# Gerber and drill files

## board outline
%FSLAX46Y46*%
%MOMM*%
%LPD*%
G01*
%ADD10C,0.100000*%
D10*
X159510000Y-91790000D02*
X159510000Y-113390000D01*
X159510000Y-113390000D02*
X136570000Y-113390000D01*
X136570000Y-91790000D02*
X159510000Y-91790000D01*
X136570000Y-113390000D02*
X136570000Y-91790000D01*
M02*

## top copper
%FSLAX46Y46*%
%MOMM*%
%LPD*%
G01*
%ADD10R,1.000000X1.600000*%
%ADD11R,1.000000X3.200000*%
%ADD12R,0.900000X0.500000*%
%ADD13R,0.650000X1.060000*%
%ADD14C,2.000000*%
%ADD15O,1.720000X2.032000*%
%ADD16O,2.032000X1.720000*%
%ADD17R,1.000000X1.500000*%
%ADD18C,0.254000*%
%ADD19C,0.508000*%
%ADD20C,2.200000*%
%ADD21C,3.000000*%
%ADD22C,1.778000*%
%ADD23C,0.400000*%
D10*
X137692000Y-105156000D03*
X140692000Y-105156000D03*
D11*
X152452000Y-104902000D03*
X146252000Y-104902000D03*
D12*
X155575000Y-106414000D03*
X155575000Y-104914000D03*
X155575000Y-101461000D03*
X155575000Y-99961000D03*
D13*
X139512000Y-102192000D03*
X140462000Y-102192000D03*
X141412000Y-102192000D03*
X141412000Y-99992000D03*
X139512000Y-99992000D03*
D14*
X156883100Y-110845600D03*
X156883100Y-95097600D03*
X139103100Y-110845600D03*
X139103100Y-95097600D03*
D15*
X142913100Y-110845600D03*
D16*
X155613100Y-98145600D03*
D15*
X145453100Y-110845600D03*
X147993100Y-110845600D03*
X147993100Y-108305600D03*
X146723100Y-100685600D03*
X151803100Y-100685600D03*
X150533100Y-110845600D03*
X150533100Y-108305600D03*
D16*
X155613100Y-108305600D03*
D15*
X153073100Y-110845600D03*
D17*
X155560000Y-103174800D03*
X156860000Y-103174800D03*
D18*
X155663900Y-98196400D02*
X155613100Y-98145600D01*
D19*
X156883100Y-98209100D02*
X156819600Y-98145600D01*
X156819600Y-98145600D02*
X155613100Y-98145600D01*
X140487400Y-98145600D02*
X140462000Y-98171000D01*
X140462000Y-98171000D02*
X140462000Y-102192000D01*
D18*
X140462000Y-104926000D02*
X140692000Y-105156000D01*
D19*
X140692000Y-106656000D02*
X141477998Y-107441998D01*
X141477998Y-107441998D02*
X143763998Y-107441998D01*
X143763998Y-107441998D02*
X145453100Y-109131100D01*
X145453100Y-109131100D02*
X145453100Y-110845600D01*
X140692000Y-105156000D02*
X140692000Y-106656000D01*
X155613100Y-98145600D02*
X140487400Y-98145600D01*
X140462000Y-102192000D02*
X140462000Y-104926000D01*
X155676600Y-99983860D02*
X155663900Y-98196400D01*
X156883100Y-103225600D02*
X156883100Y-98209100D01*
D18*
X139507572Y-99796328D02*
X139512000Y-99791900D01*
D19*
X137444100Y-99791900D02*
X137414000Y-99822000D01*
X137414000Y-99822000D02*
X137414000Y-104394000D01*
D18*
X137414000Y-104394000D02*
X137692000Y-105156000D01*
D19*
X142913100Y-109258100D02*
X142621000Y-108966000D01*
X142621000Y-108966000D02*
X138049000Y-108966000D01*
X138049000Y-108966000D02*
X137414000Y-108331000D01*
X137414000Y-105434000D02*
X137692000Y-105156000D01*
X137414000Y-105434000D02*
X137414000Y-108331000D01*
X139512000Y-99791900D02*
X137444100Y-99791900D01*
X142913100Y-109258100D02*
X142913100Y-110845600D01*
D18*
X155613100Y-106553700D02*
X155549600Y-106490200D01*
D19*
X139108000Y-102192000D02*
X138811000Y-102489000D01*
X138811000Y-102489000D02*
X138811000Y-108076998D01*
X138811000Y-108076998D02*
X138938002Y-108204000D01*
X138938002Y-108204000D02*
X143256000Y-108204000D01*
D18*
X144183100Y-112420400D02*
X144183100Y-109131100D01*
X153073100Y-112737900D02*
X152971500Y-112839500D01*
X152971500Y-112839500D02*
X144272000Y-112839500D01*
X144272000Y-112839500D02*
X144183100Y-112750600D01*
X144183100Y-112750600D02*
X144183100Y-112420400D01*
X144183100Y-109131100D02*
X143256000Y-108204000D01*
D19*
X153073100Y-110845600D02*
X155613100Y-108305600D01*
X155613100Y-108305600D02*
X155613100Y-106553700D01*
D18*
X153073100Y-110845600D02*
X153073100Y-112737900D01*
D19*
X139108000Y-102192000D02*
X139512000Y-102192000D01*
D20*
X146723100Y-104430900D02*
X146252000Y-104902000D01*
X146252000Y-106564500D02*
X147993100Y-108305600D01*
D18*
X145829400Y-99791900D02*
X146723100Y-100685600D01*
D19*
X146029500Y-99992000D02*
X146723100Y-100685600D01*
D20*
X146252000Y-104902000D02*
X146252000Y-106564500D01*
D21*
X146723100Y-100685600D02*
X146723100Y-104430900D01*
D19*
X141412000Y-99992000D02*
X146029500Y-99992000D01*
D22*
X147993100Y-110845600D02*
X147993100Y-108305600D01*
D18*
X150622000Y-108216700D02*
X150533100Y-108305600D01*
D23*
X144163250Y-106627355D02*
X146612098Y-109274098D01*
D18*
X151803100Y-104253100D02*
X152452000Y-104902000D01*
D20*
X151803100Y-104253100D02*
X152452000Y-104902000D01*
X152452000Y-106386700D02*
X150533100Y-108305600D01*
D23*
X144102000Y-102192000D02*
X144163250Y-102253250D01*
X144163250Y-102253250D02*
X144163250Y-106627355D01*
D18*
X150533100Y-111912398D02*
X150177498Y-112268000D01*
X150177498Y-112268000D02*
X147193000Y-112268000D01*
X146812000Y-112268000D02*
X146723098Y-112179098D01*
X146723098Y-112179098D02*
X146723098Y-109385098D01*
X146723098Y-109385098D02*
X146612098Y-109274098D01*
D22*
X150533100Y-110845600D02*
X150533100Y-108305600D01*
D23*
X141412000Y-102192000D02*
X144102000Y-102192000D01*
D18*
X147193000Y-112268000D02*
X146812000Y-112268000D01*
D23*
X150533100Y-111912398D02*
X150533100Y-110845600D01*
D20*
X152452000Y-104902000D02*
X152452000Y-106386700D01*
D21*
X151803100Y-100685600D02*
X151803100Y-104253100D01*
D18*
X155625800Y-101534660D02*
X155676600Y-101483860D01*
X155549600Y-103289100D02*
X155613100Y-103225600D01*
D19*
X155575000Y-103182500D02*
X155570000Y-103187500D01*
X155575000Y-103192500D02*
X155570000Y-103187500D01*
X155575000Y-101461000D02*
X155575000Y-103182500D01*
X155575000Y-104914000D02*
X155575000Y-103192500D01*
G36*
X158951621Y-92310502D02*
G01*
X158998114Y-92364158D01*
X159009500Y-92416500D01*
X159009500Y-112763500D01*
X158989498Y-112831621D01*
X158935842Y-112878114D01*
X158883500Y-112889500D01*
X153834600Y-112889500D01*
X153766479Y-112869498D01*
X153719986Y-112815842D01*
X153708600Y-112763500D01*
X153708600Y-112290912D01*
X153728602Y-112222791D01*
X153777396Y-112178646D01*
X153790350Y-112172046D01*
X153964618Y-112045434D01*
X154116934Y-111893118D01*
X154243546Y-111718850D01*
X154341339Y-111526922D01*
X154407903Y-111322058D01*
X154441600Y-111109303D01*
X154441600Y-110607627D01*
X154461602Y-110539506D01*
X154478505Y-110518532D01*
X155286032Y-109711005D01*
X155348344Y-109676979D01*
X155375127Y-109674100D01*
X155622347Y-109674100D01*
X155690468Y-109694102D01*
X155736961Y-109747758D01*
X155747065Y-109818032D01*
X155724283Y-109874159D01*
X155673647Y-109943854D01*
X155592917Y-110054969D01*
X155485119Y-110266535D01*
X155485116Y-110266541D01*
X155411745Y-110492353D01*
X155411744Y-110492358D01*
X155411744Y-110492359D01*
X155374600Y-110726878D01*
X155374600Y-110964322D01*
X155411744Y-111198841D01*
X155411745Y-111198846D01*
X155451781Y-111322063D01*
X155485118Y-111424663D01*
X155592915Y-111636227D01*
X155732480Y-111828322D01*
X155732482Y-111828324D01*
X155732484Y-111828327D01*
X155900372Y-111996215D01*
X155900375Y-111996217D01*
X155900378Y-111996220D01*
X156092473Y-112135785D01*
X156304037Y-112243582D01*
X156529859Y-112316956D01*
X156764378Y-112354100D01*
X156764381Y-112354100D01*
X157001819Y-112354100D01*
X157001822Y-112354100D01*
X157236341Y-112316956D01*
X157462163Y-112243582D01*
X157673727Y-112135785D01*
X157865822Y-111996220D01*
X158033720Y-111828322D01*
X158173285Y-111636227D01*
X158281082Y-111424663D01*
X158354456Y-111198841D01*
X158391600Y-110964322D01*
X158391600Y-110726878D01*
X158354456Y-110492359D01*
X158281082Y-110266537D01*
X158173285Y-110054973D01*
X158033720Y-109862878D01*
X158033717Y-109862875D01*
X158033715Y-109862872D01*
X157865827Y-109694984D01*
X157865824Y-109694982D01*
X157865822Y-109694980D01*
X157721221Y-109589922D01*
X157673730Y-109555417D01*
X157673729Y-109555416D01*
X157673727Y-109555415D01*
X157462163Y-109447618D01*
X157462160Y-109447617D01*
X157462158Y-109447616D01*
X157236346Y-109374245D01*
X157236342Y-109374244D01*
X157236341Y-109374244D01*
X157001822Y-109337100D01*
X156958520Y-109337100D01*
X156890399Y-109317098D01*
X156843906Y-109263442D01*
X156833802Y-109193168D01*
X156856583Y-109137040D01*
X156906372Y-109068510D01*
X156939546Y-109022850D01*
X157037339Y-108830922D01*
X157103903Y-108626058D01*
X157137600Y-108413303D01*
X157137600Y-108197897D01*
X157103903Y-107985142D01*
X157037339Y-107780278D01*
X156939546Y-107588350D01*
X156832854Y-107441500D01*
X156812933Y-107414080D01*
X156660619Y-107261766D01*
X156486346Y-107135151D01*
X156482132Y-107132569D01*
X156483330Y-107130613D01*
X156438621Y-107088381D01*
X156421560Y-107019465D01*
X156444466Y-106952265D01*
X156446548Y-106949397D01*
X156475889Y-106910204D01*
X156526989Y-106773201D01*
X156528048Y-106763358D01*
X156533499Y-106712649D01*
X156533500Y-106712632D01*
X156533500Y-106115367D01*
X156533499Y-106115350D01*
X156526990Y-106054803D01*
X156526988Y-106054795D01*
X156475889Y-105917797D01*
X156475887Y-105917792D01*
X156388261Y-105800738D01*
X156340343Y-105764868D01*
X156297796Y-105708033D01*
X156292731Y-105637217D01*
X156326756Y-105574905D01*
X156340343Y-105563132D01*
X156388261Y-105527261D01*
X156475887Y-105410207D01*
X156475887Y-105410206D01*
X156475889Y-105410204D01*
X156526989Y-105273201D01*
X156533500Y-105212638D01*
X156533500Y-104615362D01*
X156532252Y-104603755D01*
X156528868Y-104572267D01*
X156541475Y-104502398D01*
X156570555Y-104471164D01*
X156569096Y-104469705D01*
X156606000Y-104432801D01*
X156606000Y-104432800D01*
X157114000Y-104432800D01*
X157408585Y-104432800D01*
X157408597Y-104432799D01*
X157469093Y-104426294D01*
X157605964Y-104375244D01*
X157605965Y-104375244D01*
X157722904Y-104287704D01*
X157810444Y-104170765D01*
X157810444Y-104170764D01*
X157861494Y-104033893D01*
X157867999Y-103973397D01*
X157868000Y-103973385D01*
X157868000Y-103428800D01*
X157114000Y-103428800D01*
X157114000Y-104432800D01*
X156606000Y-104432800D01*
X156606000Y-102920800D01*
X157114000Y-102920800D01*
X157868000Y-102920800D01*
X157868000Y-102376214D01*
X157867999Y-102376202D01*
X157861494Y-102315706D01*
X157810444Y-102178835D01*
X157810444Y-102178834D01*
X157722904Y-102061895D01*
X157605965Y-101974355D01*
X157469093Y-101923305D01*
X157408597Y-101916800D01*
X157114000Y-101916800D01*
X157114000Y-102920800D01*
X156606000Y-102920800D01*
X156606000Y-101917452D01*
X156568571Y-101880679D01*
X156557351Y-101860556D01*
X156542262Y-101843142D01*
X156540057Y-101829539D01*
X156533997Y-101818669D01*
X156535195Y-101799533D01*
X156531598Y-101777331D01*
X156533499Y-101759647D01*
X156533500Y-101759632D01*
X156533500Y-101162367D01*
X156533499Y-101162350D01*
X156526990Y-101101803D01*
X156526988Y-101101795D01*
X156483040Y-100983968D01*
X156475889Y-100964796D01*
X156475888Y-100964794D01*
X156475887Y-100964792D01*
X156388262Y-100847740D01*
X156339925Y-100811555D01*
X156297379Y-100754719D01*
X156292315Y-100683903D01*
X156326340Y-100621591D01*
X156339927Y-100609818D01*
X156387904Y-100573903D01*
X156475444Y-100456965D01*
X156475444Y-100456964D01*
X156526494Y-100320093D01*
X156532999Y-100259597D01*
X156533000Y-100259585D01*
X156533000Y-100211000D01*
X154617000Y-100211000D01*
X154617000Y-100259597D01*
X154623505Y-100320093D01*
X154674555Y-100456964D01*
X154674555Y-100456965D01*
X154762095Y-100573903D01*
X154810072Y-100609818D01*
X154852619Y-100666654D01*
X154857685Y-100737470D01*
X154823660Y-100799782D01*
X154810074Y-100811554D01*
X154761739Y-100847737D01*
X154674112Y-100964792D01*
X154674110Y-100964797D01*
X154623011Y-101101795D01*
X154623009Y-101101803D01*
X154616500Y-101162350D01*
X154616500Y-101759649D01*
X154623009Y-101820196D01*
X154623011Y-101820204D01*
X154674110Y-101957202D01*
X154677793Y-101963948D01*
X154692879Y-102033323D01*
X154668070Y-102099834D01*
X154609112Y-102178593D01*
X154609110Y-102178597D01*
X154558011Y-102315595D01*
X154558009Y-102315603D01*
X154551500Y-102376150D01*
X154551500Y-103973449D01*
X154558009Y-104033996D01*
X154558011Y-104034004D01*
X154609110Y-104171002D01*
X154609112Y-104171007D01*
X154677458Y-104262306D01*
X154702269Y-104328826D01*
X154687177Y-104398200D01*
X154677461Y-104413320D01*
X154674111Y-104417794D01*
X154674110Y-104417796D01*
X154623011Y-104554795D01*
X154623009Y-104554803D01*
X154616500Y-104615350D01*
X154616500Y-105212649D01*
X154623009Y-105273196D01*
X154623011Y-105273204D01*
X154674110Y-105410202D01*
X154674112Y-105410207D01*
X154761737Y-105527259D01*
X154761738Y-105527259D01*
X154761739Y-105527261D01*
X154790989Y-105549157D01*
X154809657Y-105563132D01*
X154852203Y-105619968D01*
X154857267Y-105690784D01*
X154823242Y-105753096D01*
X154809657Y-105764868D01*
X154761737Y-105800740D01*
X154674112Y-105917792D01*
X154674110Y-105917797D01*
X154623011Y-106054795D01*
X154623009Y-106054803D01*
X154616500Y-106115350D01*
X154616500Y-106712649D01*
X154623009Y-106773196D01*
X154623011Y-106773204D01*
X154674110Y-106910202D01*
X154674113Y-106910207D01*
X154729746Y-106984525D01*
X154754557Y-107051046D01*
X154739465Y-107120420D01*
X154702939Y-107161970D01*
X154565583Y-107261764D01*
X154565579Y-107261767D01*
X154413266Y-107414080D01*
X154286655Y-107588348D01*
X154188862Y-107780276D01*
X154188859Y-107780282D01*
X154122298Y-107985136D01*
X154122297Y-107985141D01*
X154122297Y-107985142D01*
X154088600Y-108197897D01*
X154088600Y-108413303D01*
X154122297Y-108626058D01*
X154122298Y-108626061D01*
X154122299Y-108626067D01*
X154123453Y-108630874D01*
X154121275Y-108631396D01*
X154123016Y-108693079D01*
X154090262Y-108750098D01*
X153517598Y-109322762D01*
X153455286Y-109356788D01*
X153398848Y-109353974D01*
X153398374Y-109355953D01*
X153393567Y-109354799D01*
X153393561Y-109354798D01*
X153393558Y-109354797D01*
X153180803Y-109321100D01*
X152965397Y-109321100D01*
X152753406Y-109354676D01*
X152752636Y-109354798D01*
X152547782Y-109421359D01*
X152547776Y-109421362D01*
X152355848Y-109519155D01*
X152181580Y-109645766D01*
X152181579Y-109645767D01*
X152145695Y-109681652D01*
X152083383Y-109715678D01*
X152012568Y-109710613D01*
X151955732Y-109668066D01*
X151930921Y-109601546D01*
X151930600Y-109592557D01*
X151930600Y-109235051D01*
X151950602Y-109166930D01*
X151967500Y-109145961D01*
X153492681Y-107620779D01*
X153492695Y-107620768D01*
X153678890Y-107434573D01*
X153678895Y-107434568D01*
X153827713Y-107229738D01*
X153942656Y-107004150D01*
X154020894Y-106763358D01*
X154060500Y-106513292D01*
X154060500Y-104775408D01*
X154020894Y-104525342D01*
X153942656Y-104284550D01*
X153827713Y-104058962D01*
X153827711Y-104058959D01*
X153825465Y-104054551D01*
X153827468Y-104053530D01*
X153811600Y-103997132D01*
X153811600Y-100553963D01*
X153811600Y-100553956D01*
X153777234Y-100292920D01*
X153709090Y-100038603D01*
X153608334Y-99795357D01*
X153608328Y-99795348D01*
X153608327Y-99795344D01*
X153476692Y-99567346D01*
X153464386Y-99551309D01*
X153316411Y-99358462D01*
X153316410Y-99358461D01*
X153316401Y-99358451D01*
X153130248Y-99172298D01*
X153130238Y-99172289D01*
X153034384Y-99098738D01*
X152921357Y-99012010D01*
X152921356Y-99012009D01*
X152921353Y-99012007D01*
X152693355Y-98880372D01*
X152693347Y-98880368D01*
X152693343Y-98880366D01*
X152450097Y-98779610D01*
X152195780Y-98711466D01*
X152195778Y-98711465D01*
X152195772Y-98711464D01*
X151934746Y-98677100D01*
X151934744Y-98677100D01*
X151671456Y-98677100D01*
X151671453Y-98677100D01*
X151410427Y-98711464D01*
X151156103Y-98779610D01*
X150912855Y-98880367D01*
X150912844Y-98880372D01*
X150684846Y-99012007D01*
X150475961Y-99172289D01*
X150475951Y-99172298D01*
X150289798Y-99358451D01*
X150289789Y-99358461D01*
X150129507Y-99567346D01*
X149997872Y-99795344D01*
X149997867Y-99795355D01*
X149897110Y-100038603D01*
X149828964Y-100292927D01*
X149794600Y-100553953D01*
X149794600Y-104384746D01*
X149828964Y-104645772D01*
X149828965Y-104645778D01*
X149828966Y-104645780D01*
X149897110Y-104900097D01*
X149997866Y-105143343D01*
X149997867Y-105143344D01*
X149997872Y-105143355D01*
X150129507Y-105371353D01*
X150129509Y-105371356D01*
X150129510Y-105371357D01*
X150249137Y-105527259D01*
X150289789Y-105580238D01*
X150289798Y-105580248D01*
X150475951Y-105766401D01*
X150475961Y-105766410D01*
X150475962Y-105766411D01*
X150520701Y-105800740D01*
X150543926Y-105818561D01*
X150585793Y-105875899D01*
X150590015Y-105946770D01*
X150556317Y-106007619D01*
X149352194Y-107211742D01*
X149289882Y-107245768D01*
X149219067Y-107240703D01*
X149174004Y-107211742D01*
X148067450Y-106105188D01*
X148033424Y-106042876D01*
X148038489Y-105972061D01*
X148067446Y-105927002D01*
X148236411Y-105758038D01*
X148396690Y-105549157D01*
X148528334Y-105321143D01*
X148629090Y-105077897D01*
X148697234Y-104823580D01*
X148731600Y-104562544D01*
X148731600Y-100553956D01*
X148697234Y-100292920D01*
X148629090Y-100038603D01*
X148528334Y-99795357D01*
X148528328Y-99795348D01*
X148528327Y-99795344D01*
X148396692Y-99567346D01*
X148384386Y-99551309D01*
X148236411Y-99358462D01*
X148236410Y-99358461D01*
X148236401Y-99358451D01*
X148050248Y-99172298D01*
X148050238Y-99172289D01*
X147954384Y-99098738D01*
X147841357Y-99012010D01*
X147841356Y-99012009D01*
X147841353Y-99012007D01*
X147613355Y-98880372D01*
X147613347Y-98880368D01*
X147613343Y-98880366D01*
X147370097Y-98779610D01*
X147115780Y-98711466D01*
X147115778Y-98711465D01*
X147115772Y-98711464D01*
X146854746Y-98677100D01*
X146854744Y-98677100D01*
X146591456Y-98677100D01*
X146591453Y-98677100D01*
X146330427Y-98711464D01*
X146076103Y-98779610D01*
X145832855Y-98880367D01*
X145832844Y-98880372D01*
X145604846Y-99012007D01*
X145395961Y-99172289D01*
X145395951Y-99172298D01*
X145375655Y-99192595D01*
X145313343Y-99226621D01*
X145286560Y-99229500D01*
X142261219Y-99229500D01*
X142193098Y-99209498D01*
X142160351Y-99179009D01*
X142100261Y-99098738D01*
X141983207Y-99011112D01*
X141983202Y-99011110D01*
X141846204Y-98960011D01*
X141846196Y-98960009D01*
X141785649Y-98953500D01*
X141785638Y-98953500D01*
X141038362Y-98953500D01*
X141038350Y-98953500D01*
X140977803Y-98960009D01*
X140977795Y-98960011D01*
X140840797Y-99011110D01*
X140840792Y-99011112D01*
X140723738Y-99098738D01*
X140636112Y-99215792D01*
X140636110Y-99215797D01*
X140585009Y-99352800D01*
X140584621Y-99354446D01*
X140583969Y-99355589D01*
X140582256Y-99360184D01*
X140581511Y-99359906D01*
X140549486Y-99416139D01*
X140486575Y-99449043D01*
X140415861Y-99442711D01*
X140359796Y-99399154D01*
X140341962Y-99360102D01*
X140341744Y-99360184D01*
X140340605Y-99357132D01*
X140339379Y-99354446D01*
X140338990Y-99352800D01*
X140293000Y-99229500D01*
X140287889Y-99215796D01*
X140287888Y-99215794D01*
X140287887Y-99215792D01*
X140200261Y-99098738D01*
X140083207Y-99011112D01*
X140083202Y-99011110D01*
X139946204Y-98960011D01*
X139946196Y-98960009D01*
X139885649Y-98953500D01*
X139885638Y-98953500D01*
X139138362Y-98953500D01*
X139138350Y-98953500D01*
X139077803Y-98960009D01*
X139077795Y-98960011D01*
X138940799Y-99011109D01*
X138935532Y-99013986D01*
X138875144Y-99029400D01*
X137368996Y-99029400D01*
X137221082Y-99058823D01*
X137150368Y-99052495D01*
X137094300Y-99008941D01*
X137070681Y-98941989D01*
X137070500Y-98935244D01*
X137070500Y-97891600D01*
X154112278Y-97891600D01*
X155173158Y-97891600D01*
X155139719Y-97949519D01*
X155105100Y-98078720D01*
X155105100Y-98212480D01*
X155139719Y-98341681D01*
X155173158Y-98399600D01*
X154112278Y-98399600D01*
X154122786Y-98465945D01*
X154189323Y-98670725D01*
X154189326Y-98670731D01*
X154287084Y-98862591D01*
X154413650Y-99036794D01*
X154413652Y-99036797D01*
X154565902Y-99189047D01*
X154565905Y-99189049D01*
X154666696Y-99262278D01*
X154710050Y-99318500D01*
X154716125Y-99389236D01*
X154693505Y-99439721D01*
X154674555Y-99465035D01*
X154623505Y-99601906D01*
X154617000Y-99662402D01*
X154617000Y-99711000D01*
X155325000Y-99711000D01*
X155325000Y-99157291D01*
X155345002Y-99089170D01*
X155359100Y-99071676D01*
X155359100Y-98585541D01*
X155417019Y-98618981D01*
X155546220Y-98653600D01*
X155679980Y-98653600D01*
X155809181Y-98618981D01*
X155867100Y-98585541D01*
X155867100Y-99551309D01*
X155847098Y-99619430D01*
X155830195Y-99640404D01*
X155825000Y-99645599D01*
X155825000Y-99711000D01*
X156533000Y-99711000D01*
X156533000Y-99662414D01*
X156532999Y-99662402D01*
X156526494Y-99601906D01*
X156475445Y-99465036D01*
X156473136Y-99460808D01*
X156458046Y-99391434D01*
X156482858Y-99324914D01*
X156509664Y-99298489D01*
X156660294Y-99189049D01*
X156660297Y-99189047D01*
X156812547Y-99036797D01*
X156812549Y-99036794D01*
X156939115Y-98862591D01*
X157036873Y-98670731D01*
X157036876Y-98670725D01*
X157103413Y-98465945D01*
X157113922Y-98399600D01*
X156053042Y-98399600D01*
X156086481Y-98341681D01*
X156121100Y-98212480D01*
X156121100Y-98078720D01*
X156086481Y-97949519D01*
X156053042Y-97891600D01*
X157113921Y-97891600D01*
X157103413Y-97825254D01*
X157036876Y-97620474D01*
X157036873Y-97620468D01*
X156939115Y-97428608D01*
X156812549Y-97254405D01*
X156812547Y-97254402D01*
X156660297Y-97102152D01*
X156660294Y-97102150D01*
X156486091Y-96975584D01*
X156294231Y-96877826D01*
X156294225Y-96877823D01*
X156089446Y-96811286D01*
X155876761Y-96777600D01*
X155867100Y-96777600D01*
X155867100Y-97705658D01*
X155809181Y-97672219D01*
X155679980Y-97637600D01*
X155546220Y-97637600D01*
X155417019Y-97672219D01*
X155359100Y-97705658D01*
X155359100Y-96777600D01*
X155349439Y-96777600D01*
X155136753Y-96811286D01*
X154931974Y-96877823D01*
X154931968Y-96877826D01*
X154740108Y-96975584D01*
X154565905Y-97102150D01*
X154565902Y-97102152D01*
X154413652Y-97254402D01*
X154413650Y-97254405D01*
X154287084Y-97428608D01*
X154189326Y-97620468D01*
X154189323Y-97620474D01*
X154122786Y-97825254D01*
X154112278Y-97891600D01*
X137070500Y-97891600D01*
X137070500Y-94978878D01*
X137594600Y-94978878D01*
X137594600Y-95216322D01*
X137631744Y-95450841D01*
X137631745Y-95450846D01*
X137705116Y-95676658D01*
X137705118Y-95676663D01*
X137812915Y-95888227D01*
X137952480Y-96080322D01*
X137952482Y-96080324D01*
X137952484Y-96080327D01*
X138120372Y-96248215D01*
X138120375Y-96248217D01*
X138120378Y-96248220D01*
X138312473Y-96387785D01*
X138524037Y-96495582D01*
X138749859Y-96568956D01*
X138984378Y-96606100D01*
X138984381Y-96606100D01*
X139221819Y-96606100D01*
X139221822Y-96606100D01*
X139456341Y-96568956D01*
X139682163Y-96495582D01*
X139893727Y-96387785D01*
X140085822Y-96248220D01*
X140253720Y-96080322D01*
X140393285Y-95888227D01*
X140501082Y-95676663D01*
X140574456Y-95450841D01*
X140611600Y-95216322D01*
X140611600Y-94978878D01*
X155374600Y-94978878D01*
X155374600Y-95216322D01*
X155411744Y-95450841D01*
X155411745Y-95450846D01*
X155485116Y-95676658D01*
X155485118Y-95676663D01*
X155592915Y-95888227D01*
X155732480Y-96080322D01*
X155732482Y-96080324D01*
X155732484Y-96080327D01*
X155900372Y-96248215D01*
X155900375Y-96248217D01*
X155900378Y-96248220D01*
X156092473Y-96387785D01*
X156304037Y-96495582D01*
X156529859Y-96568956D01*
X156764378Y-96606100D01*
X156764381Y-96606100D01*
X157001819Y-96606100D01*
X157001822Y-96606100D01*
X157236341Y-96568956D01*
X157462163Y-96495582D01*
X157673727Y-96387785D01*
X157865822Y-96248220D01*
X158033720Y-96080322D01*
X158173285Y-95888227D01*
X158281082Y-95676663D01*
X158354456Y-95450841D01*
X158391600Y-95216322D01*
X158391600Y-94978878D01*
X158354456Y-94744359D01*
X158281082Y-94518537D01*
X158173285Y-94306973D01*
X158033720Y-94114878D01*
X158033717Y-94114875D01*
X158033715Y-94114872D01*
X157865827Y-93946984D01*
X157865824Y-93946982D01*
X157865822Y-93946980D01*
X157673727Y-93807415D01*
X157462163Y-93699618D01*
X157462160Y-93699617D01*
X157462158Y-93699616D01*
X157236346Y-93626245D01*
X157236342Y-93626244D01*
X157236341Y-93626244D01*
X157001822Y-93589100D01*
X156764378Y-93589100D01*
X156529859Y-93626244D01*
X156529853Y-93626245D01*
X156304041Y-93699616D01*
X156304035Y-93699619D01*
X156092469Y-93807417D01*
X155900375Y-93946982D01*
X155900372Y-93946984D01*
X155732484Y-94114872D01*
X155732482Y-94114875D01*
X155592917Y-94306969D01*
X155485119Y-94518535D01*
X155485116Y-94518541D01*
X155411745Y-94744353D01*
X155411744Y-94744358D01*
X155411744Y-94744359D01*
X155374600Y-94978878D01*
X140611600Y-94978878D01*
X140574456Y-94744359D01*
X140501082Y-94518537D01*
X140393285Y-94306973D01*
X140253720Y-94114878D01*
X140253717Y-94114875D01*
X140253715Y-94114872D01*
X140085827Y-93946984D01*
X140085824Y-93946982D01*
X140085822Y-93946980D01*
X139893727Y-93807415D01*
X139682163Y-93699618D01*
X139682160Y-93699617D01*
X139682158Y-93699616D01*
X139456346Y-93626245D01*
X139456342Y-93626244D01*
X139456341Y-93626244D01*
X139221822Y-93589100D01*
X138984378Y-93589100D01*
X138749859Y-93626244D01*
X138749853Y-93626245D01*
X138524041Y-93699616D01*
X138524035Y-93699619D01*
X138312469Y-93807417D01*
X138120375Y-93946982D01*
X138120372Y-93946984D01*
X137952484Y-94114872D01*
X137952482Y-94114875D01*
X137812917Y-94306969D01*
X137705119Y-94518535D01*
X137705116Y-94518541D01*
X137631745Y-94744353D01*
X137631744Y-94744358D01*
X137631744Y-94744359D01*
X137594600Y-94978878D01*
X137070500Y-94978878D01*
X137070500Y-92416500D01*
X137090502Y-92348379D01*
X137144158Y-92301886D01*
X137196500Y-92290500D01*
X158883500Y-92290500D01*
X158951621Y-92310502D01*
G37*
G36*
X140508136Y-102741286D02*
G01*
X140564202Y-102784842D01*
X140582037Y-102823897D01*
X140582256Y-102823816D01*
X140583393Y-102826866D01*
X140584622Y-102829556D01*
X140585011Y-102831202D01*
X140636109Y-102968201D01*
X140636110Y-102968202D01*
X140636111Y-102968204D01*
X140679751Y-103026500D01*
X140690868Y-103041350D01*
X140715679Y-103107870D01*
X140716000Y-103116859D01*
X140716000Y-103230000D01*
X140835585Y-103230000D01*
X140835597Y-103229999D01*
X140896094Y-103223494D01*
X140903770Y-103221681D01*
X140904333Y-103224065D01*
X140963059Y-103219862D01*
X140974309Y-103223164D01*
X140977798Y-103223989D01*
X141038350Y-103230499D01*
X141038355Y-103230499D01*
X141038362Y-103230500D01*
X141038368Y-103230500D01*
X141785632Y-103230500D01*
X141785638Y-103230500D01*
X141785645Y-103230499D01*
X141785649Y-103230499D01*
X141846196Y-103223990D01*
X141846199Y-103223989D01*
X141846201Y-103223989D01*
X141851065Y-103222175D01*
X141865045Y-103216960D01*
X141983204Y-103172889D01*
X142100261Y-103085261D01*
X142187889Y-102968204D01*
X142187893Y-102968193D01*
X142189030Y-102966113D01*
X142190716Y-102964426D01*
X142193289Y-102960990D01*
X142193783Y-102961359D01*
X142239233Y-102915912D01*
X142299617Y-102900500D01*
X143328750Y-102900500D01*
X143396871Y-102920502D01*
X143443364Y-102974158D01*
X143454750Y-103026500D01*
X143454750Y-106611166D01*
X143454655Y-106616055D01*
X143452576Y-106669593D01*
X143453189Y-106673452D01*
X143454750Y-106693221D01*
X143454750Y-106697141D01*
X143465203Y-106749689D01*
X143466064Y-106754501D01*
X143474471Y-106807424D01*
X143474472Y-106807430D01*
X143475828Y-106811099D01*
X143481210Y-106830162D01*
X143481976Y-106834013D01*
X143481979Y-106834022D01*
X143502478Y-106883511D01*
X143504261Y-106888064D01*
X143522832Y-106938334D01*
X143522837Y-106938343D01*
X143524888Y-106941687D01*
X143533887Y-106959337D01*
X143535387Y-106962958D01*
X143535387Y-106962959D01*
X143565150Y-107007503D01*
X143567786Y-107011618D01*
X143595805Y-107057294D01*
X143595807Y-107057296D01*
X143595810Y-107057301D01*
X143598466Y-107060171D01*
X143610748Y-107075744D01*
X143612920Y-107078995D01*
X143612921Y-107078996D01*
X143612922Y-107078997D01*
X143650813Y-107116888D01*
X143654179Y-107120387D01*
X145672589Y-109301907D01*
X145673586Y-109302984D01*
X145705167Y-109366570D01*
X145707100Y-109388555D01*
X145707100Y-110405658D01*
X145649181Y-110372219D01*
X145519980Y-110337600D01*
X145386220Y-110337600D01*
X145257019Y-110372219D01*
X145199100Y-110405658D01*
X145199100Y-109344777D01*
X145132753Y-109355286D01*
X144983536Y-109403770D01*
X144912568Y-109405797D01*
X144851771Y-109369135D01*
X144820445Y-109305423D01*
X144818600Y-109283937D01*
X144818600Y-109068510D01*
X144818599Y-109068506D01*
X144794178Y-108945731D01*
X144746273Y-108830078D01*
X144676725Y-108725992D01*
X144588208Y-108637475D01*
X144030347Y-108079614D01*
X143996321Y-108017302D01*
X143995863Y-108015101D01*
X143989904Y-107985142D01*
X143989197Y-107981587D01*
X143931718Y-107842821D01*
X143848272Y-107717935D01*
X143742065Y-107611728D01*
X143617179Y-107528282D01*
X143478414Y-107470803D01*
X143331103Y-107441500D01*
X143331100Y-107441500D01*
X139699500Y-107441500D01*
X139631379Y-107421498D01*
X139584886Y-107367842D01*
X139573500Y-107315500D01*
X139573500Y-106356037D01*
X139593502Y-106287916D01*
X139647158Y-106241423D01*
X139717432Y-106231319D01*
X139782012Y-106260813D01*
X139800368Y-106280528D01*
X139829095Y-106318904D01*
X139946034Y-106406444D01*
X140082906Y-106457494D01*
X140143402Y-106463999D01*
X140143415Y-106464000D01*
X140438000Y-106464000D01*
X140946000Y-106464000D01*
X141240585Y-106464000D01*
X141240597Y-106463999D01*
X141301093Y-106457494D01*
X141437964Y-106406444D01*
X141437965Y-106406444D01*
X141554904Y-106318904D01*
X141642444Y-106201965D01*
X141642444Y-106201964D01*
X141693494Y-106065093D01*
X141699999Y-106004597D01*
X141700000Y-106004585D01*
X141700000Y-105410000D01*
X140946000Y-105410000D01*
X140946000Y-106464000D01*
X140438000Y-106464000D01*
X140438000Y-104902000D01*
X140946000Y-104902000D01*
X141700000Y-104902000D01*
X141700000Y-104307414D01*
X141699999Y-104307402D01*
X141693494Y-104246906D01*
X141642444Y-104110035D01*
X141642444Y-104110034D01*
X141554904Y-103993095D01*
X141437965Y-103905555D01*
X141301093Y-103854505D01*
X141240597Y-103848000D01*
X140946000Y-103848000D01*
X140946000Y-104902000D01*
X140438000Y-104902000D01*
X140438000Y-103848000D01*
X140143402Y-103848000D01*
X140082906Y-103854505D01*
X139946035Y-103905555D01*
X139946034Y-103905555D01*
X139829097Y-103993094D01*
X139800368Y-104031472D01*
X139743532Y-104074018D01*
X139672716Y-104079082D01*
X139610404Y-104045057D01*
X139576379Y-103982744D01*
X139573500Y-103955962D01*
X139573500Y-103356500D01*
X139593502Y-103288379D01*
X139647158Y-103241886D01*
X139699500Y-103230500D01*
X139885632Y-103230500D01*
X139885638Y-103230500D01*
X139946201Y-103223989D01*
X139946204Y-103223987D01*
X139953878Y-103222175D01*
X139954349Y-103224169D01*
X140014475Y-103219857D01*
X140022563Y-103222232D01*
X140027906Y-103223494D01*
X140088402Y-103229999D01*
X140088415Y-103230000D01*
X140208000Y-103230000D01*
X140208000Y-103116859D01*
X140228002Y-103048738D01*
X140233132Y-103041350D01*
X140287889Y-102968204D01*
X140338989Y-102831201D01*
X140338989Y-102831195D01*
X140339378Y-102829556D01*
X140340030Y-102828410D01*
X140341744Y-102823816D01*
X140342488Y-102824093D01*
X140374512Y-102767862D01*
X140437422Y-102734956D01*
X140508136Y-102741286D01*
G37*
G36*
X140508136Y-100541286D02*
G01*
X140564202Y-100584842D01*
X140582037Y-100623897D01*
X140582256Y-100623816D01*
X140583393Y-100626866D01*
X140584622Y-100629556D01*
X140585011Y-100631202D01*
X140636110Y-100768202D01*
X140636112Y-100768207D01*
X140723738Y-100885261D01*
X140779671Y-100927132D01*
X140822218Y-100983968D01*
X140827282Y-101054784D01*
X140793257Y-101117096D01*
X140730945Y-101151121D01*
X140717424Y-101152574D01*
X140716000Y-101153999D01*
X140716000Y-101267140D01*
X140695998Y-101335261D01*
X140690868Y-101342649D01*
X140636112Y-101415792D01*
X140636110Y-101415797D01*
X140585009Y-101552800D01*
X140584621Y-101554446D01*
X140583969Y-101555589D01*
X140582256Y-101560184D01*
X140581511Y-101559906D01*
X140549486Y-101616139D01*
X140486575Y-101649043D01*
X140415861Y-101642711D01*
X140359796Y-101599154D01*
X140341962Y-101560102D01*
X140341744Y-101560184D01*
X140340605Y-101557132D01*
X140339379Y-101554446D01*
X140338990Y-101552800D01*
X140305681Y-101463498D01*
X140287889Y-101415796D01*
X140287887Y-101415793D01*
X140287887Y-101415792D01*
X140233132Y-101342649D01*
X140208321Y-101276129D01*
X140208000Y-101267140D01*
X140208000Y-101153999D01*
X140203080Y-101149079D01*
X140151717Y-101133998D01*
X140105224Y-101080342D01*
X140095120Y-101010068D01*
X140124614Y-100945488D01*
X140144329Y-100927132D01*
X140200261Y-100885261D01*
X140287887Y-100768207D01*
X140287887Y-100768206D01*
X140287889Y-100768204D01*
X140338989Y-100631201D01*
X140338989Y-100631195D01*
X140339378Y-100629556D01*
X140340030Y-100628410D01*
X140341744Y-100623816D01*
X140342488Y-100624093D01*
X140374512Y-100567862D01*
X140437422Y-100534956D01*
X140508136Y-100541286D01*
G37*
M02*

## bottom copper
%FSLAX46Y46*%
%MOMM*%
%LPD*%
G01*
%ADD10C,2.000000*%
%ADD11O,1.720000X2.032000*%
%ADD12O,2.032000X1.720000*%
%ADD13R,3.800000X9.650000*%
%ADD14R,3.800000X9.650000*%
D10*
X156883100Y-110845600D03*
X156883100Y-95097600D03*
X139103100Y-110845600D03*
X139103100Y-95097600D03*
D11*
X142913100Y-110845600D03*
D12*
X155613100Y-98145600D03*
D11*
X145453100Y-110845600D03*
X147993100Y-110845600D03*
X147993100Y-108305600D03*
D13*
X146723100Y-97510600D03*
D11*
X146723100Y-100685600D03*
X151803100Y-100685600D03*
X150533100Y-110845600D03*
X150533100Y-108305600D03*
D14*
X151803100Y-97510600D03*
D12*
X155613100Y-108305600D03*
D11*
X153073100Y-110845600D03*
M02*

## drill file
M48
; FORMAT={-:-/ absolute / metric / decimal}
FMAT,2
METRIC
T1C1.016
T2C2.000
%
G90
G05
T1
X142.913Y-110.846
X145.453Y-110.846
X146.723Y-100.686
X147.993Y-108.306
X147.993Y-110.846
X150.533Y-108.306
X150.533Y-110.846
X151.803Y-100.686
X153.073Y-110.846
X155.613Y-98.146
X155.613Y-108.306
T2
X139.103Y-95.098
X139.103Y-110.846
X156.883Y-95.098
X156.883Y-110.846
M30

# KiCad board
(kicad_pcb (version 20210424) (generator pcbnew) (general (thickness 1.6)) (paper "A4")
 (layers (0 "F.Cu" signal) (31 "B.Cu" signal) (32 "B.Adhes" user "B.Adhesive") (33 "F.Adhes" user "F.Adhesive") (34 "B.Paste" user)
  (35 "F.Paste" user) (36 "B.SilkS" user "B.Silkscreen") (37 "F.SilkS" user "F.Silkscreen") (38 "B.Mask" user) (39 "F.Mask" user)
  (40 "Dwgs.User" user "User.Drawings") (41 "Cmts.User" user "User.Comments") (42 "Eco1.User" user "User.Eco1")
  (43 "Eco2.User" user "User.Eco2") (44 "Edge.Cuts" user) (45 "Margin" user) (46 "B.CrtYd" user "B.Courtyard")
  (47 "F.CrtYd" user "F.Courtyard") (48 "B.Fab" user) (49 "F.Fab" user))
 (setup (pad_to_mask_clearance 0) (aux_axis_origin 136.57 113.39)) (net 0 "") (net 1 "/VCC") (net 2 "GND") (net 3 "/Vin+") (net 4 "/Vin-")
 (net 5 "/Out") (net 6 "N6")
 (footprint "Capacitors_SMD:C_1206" (layer "F.Cu") (at 139.192 105.156)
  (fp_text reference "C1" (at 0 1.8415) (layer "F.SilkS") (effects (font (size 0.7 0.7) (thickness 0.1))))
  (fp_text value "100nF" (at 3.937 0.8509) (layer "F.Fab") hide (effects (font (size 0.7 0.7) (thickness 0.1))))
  (pad "1" smd rect locked (at -1.5 0) (size 1 1.6) (layers "F.Cu" "F.Paste" "F.Mask") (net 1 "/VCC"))
  (pad "2" smd rect locked (at 1.5 0) (size 1 1.6) (layers "F.Cu" "F.Paste" "F.Mask") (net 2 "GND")))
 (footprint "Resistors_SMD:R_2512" (layer "F.Cu") (at 149.352 104.902 180)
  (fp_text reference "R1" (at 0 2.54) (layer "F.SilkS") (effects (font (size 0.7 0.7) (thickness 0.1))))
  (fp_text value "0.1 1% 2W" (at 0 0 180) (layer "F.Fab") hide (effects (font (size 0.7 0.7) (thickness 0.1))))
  (pad "1" smd rect locked (at -3.1 0 180) (size 1 3.2) (layers "F.Cu" "F.Paste" "F.Mask") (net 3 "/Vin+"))
  (pad "2" smd rect locked (at 3.1 0 180) (size 1 3.2) (layers "F.Cu" "F.Paste" "F.Mask") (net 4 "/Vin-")))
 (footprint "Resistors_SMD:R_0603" (layer "F.Cu") (at 155.575 105.664 90)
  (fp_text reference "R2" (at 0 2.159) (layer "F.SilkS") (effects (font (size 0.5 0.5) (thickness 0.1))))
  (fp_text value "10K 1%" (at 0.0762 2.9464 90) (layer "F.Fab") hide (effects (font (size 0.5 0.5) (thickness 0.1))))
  (pad "1" smd rect locked (at -0.75 0 90) (size 0.5 0.9) (layers "F.Cu" "F.Paste" "F.Mask") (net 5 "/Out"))
  (pad "2" smd rect locked (at 0.75 0 90) (size 0.5 0.9) (layers "F.Cu" "F.Paste" "F.Mask") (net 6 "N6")))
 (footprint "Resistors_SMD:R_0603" (layer "F.Cu") (at 155.575 100.711 90)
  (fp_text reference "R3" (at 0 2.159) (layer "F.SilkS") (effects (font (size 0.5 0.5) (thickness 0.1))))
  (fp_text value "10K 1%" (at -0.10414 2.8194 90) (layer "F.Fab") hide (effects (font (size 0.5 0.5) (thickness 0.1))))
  (pad "1" smd rect locked (at -0.75 0 90) (size 0.5 0.9) (layers "F.Cu" "F.Paste" "F.Mask") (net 6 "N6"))
  (pad "2" smd rect locked (at 0.75 0 90) (size 0.5 0.9) (layers "F.Cu" "F.Paste" "F.Mask") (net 2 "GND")))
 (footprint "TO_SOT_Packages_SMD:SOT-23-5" (layer "F.Cu") (at 140.462 101.092 90)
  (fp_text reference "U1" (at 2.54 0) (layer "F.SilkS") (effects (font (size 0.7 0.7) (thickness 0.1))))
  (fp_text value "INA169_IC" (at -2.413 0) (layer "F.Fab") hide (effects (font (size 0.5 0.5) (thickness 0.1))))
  (pad "1" smd rect locked (at -1.1 -0.95 90) (size 1.06 0.65) (layers "F.Cu" "F.Paste" "F.Mask") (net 5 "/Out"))
  (pad "2" smd rect locked (at -1.1 0 90) (size 1.06 0.65) (layers "F.Cu" "F.Paste" "F.Mask") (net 2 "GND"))
  (pad "3" smd rect locked (at -1.1 0.95 90) (size 1.06 0.65) (layers "F.Cu" "F.Paste" "F.Mask") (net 3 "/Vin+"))
  (pad "4" smd rect locked (at 1.1 0.95 90) (size 1.06 0.65) (layers "F.Cu" "F.Paste" "F.Mask") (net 4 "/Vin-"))
  (pad "5" smd rect locked (at 1.1 -0.95 90) (size 1.06 0.65) (layers "F.Cu" "F.Paste" "F.Mask") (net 1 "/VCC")))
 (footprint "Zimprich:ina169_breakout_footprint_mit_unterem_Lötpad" (layer "F.Cu") (at 147.9931 103.2256)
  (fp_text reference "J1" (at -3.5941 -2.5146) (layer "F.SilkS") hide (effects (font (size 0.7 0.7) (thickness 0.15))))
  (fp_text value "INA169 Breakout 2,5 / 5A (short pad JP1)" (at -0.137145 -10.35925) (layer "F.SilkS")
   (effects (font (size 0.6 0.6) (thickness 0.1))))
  (pad "" thru_hole circle locked (at 8.89 7.62) (size 2 2) (drill 2) (layers *.Cu *.Mask "F.SilkS"))
  (pad "" thru_hole circle locked (at 8.89 -8.128) (size 2 2) (drill 2) (layers *.Cu *.Mask "F.SilkS"))
  (pad "" thru_hole circle locked (at -8.89 7.62) (size 2 2) (drill 2) (layers *.Cu *.Mask "F.SilkS"))
  (pad "" thru_hole circle locked (at -8.89 -8.128) (size 2 2) (drill 2) (layers *.Cu *.Mask "F.SilkS"))
  (pad "1" thru_hole oval locked (at -5.08 7.62) (size 1.72 2.032) (drill 1.016) (layers *.Cu *.Mask) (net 1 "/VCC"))
  (pad "2" thru_hole oval locked (at 7.62 -5.08) (size 2.032 1.72) (drill 1.016) (layers *.Cu *.Mask) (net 2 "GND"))
  (pad "2" thru_hole oval locked (at -2.54 7.62) (size 1.72 2.032) (drill 1.016) (layers *.Cu *.Mask) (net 2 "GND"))
  (pad "3" thru_hole oval locked (at 0 7.62) (size 1.72 2.032) (drill 1.016) (layers *.Cu *.Mask) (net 4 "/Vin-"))
  (pad "3" thru_hole oval locked (at 0 5.08) (size 1.72 2.032) (drill 1.016) (layers *.Cu *.Mask) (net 4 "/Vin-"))
  (pad "3" connect rect locked (at -1.27 -5.715) (size 3.8 9.65) (layers "B.Cu" "B.Mask") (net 4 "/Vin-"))
  (pad "3" thru_hole oval locked (at -1.27 -2.54) (size 1.72 2.032) (drill 1.016) (layers *.Cu *.Mask) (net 4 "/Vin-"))
  (pad "4" thru_hole oval locked (at 3.81 -2.54) (size 1.72 2.032) (drill 1.016) (layers *.Cu *.Mask) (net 3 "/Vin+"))
  (pad "4" thru_hole oval locked (at 2.54 7.62) (size 1.72 2.032) (drill 1.016) (layers *.Cu *.Mask) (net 3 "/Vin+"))
  (pad "4" thru_hole oval locked (at 2.54 5.08) (size 1.72 2.032) (drill 1.016) (layers *.Cu *.Mask) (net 3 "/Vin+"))
  (pad "4" smd rect locked (at 3.81 -5.715) (size 3.8 9.65) (layers "B.Cu" "B.Mask") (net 3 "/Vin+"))
  (pad "5" thru_hole oval locked (at 7.62 5.08) (size 2.032 1.72) (drill 1.016) (layers *.Cu *.Mask) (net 5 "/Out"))
  (pad "5" thru_hole oval locked (at 5.08 7.62) (size 1.72 2.032) (drill 1.016) (layers *.Cu *.Mask) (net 5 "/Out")))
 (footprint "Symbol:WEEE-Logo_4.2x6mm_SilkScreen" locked (layer "F.Cu") (at 143.129 106.172)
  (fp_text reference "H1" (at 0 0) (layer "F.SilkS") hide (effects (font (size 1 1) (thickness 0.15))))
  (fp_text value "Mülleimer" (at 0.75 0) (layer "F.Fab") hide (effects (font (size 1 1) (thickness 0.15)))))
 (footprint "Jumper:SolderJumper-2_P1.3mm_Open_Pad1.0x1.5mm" (layer "F.Cu") (at 156.21 103.1748)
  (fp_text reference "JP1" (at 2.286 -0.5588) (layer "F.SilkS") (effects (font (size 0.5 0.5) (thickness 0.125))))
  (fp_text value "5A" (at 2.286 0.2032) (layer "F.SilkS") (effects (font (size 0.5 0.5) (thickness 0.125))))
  (pad "1" smd rect locked (at -0.65 0) (size 1 1.5) (layers "F.Cu" "F.Mask") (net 6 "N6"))
  (pad "2" smd rect locked (at 0.65 0) (size 1 1.5) (layers "F.Cu" "F.Mask") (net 2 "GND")))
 (gr_line (start 159.51 91.79) (end 159.51 113.39) (angle 90) (layer "Edge.Cuts") (width 0.1))
 (gr_line (start 159.51 113.39) (end 136.57 113.39) (angle 90) (layer "Edge.Cuts") (width 0.1))
 (gr_line (start 136.57 91.79) (end 159.51 91.79) (angle 90) (layer "Edge.Cuts") (width 0.1))
 (gr_line (start 136.57 113.39) (end 136.57 91.79) (angle 90) (layer "Edge.Cuts") (width 0.1))
 (segment (start 155.6639 98.1964) (end 155.6131 98.1456) (width 0.254) (layer "F.Cu") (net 2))
 (segment (start 156.8831 98.2091) (end 156.8196 98.1456) (width 0.508) (layer "F.Cu") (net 2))
 (segment (start 156.8196 98.1456) (end 155.6131 98.1456) (width 0.508) (layer "F.Cu") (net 2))
 (segment (start 140.4874 98.1456) (end 140.462 98.171) (width 0.508) (layer "F.Cu") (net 2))
 (segment (start 140.462 98.171) (end 140.462 102.192) (width 0.508) (layer "F.Cu") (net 2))
 (segment (start 140.462 104.926) (end 140.692 105.156) (width 0.254) (layer "F.Cu") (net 2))
 (segment (start 140.692 106.656) (end 141.477998 107.441998) (width 0.508) (layer "F.Cu") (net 2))
 (segment (start 141.477998 107.441998) (end 143.763998 107.441998) (width 0.508) (layer "F.Cu") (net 2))
 (segment (start 143.763998 107.441998) (end 145.4531 109.1311) (width 0.508) (layer "F.Cu") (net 2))
 (segment (start 145.4531 109.1311) (end 145.4531 110.8456) (width 0.508) (layer "F.Cu") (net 2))
 (segment (start 140.692 105.156) (end 140.692 106.656) (width 0.508) (layer "F.Cu") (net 2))
 (segment (start 155.6131 98.1456) (end 140.4874 98.1456) (width 0.508) (layer "F.Cu") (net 2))
 (segment (start 140.462 102.192) (end 140.462 104.926) (width 0.508) (layer "F.Cu") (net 2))
 (segment (start 155.6766 99.98386) (end 155.6639 98.1964) (width 0.508) (layer "F.Cu") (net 2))
 (segment (start 156.8831 103.2256) (end 156.8831 98.2091) (width 0.508) (layer "F.Cu") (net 2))
 (segment (start 139.507572 99.796328) (end 139.512 99.7919) (width 0.254) (layer "F.Cu") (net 1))
 (segment (start 137.4441 99.7919) (end 137.414 99.822) (width 0.508) (layer "F.Cu") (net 1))
 (segment (start 137.414 99.822) (end 137.414 104.394) (width 0.508) (layer "F.Cu") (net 1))
 (segment (start 137.414 104.394) (end 137.692 105.156) (width 0.254) (layer "F.Cu") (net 1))
 (segment (start 142.9131 109.2581) (end 142.621 108.966) (width 0.508) (layer "F.Cu") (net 1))
 (segment (start 142.621 108.966) (end 138.049 108.966) (width 0.508) (layer "F.Cu") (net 1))
 (segment (start 138.049 108.966) (end 137.414 108.331) (width 0.508) (layer "F.Cu") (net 1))
 (segment (start 137.414 105.434) (end 137.692 105.156) (width 0.508) (layer "F.Cu") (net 1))
 (segment (start 137.414 105.434) (end 137.414 108.331) (width 0.508) (layer "F.Cu") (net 1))
 (segment (start 139.512 99.7919) (end 137.4441 99.7919) (width 0.508) (layer "F.Cu") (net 1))
 (segment (start 142.9131 109.2581) (end 142.9131 110.8456) (width 0.508) (layer "F.Cu") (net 1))
 (segment (start 155.6131 106.5537) (end 155.5496 106.4902) (width 0.254) (layer "F.Cu") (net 5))
 (segment (start 139.108 102.192) (end 138.811 102.489) (width 0.508) (layer "F.Cu") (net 5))
 (segment (start 138.811 102.489) (end 138.811 108.076998) (width 0.508) (layer "F.Cu") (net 5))
 (segment (start 138.811 108.076998) (end 138.938002 108.204) (width 0.508) (layer "F.Cu") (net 5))
 (segment (start 138.938002 108.204) (end 143.256 108.204) (width 0.508) (layer "F.Cu") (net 5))
 (segment (start 144.1831 112.4204) (end 144.1831 109.1311) (width 0.254) (layer "F.Cu") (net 5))
 (segment (start 153.0731 112.7379) (end 152.9715 112.8395) (width 0.254) (layer "F.Cu") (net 5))
 (segment (start 152.9715 112.8395) (end 144.272 112.8395) (width 0.254) (layer "F.Cu") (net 5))
 (segment (start 144.272 112.8395) (end 144.1831 112.7506) (width 0.254) (layer "F.Cu") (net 5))
 (segment (start 144.1831 112.7506) (end 144.1831 112.4204) (width 0.254) (layer "F.Cu") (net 5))
 (segment (start 144.1831 109.1311) (end 143.256 108.204) (width 0.254) (layer "F.Cu") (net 5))
 (segment (start 153.0731 110.8456) (end 155.6131 108.3056) (width 0.508) (layer "F.Cu") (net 5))
 (segment (start 155.6131 108.3056) (end 155.6131 106.5537) (width 0.508) (layer "F.Cu") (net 5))
 (segment (start 153.0731 110.8456) (end 153.0731 112.7379) (width 0.254) (layer "F.Cu") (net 5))
 (segment (start 139.108 102.192) (end 139.512 102.192) (width 0.508) (layer "F.Cu") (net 5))
 (segment (start 146.7231 104.4309) (end 146.252 104.902) (width 2.2) (layer "F.Cu") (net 4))
 (segment (start 146.252 106.5645) (end 147.9931 108.3056) (width 2.2) (layer "F.Cu") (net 4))
 (segment (start 145.8294 99.7919) (end 146.7231 100.6856) (width 0.254) (layer "F.Cu") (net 4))
 (segment (start 146.0295 99.992) (end 146.7231 100.6856) (width 0.508) (layer "F.Cu") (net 4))
 (segment (start 146.252 104.902) (end 146.252 106.5645) (width 2.2) (layer "F.Cu") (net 4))
 (segment (start 146.7231 100.6856) (end 146.7231 104.4309) (width 3) (layer "F.Cu") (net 4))
 (segment (start 141.412 99.992) (end 146.0295 99.992) (width 0.508) (layer "F.Cu") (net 4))
 (segment (start 147.9931 110.8456) (end 147.9931 108.3056) (width 1.778) (layer "F.Cu") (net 4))
 (segment (start 150.622 108.2167) (end 150.5331 108.3056) (width 0.254) (layer "F.Cu") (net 3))
 (segment (start 144.16325 106.627355) (end 146.612098 109.274098) (width 0.4) (layer "F.Cu") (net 3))
 (segment (start 151.8031 104.2531) (end 152.452 104.902) (width 0.254) (layer "F.Cu") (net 3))
 (segment (start 151.8031 104.2531) (end 152.452 104.902) (width 2.2) (layer "F.Cu") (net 3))
 (segment (start 152.452 106.3867) (end 150.5331 108.3056) (width 2.2) (layer "F.Cu") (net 3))
 (segment (start 144.102 102.192) (end 144.16325 102.25325) (width 0.4) (layer "F.Cu") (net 3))
 (segment (start 144.16325 102.25325) (end 144.16325 106.627355) (width 0.4) (layer "F.Cu") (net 3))
 (segment (start 150.5331 111.912398) (end 150.177498 112.268) (width 0.254) (layer "F.Cu") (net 3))
 (segment (start 150.177498 112.268) (end 147.193 112.268) (width 0.254) (layer "F.Cu") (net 3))
 (segment (start 146.812 112.268) (end 146.723098 112.179098) (width 0.254) (layer "F.Cu") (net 3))
 (segment (start 146.723098 112.179098) (end 146.723098 109.385098) (width 0.254) (layer "F.Cu") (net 3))
 (segment (start 146.723098 109.385098) (end 146.612098 109.274098) (width 0.254) (layer "F.Cu") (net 3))
 (segment (start 150.5331 110.8456) (end 150.5331 108.3056) (width 1.778) (layer "F.Cu") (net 3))
 (segment (start 141.412 102.192) (end 144.102 102.192) (width 0.4) (layer "F.Cu") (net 3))
 (segment (start 147.193 112.268) (end 146.812 112.268) (width 0.254) (layer "F.Cu") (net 3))
 (segment (start 150.5331 111.912398) (end 150.5331 110.8456) (width 0.4) (layer "F.Cu") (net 3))
 (segment (start 152.452 104.902) (end 152.452 106.3867) (width 2.2) (layer "F.Cu") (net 3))
 (segment (start 151.8031 100.6856) (end 151.8031 104.2531) (width 3) (layer "F.Cu") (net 3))
 (segment (start 155.6258 101.53466) (end 155.6766 101.48386) (width 0.254) (layer "F.Cu") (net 6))
 (segment (start 155.5496 103.2891) (end 155.6131 103.2256) (width 0.254) (layer "F.Cu") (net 6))
 (segment (start 155.575 103.1825) (end 155.57 103.1875) (width 0.508) (layer "F.Cu") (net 6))
 (segment (start 155.575 103.1925) (end 155.57 103.1875) (width 0.508) (layer "F.Cu") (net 6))
 (segment (start 155.575 101.461) (end 155.575 103.1825) (width 0.508) (layer "F.Cu") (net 6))
 (segment (start 155.575 104.914) (end 155.575 103.1925) (width 0.508) (layer "F.Cu") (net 6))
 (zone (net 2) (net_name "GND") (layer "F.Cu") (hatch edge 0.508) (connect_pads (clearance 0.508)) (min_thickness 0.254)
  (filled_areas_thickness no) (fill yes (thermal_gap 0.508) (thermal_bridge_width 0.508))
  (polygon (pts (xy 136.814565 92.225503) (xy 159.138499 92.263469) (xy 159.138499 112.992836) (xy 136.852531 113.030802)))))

